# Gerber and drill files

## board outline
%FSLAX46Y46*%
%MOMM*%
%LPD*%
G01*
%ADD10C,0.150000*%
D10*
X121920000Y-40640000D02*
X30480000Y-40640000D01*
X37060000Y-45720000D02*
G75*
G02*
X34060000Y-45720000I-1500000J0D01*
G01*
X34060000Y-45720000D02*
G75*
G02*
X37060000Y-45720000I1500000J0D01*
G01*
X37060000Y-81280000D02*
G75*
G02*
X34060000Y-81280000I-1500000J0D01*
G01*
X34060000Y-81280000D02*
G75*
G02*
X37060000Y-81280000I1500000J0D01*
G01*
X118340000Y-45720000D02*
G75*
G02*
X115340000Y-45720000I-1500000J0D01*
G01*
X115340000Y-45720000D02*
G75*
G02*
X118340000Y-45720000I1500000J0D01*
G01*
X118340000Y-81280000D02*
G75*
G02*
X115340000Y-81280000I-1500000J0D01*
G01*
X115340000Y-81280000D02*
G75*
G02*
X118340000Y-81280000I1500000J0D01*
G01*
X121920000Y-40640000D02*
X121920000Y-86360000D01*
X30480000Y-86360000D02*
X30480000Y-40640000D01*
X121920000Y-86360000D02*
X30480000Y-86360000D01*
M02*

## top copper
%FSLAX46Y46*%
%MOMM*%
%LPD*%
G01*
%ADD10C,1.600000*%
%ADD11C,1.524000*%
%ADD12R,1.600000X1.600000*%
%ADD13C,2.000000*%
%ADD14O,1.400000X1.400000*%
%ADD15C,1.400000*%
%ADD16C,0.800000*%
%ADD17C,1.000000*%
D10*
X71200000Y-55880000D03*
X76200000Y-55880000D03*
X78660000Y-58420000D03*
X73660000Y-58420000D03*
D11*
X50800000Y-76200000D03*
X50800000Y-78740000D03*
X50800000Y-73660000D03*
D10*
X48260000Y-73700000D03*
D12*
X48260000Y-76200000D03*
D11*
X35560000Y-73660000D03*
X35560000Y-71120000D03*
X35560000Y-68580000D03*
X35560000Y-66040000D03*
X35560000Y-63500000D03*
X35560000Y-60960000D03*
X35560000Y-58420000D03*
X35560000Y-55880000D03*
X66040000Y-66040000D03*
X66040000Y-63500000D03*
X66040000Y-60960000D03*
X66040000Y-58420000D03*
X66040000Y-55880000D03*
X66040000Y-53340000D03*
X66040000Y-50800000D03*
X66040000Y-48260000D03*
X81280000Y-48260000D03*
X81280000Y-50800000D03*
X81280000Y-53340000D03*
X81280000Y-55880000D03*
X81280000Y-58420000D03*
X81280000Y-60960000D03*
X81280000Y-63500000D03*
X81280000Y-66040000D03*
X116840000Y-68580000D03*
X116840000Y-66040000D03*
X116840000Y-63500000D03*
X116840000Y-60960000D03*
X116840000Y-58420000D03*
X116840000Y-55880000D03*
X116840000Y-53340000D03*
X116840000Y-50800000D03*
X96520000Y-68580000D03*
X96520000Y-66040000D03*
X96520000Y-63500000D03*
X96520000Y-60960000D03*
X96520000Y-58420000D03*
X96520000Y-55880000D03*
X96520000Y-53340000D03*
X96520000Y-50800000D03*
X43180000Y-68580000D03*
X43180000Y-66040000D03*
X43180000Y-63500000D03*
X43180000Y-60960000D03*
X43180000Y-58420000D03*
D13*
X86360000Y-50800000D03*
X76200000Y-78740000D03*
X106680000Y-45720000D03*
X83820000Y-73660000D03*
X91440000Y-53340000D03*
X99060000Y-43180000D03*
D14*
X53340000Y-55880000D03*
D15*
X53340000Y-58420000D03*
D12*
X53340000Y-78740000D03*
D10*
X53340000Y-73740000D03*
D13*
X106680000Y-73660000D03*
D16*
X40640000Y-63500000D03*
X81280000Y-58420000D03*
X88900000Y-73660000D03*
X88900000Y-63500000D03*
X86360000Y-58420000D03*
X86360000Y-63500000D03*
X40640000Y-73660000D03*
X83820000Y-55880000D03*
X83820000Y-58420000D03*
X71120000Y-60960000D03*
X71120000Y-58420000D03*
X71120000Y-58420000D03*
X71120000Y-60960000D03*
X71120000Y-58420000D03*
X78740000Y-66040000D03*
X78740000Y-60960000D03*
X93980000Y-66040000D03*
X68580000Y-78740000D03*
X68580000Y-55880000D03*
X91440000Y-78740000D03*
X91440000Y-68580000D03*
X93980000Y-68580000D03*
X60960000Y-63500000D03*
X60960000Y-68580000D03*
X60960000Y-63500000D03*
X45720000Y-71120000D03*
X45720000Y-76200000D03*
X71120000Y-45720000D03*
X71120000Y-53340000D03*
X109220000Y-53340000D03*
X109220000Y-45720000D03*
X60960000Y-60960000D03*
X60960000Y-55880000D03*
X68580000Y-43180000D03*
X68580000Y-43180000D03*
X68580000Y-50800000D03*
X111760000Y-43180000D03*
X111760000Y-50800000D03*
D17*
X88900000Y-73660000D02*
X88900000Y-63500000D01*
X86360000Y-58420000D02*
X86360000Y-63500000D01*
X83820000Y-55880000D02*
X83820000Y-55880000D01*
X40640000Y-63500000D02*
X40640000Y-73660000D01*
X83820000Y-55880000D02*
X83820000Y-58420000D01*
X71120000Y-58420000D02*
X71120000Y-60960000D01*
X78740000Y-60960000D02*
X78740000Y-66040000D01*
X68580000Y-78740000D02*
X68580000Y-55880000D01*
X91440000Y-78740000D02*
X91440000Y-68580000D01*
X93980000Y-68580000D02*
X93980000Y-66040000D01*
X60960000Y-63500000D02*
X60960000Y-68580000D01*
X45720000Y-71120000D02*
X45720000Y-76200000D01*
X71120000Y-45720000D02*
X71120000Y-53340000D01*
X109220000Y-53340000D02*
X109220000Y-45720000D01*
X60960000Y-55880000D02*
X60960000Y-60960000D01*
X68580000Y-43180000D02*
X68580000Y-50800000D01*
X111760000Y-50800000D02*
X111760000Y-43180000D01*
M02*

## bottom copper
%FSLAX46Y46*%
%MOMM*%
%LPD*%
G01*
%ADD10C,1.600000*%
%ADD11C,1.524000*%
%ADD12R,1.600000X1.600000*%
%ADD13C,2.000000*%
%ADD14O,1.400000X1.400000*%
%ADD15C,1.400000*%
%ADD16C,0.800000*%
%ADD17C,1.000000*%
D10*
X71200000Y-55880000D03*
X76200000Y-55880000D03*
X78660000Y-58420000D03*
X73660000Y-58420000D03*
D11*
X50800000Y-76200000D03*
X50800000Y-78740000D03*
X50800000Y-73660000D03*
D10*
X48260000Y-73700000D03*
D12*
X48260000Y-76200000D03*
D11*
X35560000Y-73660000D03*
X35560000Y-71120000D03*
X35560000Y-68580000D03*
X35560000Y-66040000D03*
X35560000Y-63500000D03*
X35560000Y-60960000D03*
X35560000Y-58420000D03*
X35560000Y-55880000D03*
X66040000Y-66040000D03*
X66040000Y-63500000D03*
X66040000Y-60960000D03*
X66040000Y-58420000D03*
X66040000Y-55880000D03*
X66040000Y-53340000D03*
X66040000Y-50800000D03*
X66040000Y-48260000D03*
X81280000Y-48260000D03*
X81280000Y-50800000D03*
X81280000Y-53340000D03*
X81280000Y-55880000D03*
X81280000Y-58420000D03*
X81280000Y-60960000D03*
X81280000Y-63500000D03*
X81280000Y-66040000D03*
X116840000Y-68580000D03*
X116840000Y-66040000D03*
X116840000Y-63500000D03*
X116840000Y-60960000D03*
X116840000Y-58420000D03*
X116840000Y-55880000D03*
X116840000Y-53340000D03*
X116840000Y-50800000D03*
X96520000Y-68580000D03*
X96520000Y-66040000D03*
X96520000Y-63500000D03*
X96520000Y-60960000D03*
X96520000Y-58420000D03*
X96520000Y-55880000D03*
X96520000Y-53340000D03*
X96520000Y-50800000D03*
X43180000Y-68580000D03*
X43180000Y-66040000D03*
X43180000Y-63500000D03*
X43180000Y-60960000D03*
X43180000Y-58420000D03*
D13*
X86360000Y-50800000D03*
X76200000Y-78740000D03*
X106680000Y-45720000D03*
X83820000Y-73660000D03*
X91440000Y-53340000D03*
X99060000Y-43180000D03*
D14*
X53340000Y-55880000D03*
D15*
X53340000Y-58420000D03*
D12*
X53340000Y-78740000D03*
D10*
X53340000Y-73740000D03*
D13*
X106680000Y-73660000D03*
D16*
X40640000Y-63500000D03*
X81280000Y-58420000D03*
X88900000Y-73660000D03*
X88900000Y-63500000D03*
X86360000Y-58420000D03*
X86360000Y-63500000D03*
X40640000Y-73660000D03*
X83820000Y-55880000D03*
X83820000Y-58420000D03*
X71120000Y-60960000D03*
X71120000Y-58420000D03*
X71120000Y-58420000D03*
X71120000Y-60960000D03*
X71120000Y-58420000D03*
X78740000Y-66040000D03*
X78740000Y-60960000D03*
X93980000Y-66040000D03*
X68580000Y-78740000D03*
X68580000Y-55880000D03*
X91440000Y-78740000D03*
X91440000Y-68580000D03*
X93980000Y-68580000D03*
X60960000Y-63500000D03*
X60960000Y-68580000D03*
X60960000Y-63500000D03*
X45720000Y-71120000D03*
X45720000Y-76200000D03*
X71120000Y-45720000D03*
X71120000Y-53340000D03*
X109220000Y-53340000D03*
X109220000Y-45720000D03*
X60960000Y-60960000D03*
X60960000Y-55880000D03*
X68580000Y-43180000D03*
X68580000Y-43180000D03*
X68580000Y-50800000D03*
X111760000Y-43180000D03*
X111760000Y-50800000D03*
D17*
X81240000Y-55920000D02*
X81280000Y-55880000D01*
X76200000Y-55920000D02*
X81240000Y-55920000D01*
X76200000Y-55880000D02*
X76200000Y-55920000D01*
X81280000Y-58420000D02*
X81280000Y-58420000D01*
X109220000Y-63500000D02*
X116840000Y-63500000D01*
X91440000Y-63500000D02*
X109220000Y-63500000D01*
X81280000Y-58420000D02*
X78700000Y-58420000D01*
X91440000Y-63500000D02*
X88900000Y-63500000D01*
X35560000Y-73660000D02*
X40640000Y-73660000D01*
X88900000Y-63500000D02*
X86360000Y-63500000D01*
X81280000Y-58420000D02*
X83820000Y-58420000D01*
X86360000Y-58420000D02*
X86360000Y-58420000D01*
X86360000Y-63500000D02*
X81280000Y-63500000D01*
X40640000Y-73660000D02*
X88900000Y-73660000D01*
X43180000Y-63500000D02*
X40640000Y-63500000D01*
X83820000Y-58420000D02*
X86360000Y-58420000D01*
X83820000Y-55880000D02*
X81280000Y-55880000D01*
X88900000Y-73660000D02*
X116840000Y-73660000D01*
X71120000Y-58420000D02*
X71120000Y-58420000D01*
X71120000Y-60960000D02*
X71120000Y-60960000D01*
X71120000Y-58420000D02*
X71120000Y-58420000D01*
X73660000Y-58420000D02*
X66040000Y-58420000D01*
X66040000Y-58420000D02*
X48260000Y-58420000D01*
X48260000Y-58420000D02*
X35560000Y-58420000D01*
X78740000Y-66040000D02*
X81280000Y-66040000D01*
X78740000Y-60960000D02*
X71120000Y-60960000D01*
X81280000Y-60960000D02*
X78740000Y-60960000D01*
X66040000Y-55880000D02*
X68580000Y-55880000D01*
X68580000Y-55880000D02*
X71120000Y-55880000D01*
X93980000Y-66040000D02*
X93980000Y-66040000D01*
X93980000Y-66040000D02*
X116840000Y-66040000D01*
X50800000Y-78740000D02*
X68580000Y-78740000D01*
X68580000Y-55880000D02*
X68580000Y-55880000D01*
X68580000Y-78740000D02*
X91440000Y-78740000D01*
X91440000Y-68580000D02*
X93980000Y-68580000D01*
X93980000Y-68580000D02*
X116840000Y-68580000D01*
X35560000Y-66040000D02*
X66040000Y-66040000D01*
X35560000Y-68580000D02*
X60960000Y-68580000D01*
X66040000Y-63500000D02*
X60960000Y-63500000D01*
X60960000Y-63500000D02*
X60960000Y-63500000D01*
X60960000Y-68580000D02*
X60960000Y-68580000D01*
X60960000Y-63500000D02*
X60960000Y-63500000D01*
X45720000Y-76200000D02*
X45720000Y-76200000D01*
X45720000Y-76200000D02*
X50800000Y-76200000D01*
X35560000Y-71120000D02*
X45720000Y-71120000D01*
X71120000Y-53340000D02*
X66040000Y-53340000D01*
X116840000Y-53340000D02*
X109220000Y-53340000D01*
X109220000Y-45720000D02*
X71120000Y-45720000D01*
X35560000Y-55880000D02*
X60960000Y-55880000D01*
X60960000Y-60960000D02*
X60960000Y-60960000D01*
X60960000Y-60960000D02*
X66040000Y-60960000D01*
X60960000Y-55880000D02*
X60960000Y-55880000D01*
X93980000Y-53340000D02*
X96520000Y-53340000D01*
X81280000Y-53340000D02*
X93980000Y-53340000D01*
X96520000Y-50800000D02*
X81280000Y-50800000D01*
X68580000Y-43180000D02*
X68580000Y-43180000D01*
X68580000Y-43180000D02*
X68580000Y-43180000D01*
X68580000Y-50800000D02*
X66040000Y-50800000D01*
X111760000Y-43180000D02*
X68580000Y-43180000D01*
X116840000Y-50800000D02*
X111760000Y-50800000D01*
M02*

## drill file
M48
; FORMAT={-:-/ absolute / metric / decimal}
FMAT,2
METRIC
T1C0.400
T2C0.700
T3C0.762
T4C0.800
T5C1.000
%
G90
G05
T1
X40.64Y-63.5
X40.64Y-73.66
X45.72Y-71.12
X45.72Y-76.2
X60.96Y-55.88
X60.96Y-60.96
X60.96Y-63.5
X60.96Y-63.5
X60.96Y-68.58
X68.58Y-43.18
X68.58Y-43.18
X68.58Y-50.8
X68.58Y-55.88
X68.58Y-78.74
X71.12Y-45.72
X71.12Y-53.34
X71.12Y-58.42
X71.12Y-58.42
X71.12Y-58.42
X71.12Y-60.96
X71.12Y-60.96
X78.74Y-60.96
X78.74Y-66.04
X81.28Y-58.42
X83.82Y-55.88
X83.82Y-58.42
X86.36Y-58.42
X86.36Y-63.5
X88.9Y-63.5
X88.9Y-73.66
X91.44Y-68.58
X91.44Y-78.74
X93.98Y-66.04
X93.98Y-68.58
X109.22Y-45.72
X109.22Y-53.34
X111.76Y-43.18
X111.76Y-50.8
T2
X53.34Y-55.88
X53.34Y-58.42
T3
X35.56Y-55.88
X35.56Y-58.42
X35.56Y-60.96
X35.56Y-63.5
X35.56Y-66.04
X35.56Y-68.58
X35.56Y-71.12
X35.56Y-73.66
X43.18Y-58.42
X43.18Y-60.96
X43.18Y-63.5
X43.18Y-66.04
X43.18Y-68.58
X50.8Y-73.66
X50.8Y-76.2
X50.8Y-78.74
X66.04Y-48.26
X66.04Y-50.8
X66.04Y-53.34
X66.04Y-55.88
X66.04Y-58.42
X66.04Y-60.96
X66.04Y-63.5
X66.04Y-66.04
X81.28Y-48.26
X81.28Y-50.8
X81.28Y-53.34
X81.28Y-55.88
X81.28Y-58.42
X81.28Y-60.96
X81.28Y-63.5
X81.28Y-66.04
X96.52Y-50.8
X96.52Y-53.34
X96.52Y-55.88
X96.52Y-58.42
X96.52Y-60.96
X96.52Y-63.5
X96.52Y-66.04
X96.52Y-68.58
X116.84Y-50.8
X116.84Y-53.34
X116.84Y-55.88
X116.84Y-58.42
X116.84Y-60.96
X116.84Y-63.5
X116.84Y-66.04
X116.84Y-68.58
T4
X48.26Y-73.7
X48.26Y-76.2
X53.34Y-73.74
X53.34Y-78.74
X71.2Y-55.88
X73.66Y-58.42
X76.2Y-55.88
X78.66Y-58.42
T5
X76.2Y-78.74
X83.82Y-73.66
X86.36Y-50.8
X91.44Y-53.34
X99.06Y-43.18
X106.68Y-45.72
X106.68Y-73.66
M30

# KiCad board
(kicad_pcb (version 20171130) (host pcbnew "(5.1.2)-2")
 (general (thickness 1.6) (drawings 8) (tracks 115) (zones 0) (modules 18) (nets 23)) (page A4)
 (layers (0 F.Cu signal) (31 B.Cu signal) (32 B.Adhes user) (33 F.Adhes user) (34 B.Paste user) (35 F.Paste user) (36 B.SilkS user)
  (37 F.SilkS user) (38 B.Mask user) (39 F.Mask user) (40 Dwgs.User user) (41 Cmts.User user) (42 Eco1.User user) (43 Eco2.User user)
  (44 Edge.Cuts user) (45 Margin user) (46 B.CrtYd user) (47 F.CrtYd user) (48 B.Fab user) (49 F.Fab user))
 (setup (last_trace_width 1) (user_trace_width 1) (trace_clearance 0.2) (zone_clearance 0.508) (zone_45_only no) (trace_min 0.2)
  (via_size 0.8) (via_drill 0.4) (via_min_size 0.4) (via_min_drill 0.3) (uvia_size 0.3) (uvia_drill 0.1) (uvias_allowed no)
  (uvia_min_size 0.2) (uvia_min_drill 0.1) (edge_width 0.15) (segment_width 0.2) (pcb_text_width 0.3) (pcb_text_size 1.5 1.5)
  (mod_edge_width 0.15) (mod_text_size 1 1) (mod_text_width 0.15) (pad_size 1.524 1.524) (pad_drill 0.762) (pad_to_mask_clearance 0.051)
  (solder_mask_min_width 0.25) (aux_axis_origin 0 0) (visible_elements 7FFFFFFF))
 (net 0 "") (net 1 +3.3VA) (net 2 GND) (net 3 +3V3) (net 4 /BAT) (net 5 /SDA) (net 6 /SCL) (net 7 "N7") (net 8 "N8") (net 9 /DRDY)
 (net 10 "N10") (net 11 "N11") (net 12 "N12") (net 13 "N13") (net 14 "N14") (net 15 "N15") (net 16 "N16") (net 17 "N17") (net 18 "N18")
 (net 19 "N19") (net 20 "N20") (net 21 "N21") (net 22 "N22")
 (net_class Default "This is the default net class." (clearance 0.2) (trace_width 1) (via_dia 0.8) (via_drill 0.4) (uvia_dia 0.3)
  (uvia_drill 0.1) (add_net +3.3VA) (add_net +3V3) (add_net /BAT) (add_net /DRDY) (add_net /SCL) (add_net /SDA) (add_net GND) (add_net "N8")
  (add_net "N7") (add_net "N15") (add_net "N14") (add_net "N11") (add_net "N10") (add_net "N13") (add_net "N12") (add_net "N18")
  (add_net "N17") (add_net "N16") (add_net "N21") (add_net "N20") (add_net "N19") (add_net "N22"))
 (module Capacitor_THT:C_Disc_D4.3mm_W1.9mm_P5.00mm (layer F.Cu) (at 76.2 55.88 180)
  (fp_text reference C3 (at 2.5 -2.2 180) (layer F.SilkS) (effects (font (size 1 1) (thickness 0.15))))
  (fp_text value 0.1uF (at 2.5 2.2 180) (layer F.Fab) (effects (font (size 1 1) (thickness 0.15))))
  (pad 2 thru_hole circle (at 5 0 180) (size 1.6 1.6) (drill 0.8) (layers *.Cu *.Mask) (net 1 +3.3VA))
  (pad 1 thru_hole circle (at 0 0 180) (size 1.6 1.6) (drill 0.8) (layers *.Cu *.Mask) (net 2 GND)))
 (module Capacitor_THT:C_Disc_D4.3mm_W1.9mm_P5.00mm (layer F.Cu) (at 73.66 58.42)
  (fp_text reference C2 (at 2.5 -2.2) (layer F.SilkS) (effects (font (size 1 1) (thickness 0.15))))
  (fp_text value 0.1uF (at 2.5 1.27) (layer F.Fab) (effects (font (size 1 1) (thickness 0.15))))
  (pad 2 thru_hole circle (at 5 0) (size 1.6 1.6) (drill 0.8) (layers *.Cu *.Mask) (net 2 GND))
  (pad 1 thru_hole circle (at 0 0) (size 1.6 1.6) (drill 0.8) (layers *.Cu *.Mask) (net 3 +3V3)))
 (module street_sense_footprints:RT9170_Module (layer F.Cu) (at 53.34 76.2 270)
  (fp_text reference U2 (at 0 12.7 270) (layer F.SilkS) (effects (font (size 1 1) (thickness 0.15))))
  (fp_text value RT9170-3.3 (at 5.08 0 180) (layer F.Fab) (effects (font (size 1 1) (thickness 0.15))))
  (pad 3 thru_hole circle (at 0 2.54 270) (size 1.524 1.524) (drill 0.762) (layers *.Cu *.Mask) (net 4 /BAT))
  (pad 2 thru_hole circle (at 2.54 2.54 270) (size 1.524 1.524) (drill 0.762) (layers *.Cu *.Mask) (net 1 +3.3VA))
  (pad 1 thru_hole circle (at -2.54 2.54 270) (size 1.524 1.524) (drill 0.762) (layers *.Cu *.Mask) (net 2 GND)))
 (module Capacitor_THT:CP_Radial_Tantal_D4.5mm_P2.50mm (layer F.Cu) (at 48.26 76.2 90)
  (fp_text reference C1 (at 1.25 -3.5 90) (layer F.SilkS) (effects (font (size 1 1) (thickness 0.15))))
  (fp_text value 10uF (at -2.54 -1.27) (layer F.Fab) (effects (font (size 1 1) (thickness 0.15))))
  (pad 2 thru_hole circle (at 2.5 0 90) (size 1.6 1.6) (drill 0.8) (layers *.Cu *.Mask) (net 2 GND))
  (pad 1 thru_hole rect (at 0 0 90) (size 1.6 1.6) (drill 0.8) (layers *.Cu *.Mask) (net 4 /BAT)))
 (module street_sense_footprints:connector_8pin (layer F.Cu) (at 35.56 53.34)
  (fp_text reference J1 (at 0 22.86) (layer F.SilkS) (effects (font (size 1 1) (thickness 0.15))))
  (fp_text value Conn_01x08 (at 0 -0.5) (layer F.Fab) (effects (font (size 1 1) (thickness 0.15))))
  (pad 8 thru_hole circle (at 0 20.32) (size 1.524 1.524) (drill 0.762) (layers *.Cu *.Mask) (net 2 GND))
  (pad 7 thru_hole circle (at 0 17.78) (size 1.524 1.524) (drill 0.762) (layers *.Cu *.Mask) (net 4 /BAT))
  (pad 6 thru_hole circle (at 0 15.24) (size 1.524 1.524) (drill 0.762) (layers *.Cu *.Mask) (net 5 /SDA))
  (pad 5 thru_hole circle (at 0 12.7) (size 1.524 1.524) (drill 0.762) (layers *.Cu *.Mask) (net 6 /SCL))
  (pad 4 thru_hole circle (at 0 10.16) (size 1.524 1.524) (drill 0.762) (layers *.Cu *.Mask) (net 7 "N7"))
  (pad 3 thru_hole circle (at 0 7.62) (size 1.524 1.524) (drill 0.762) (layers *.Cu *.Mask) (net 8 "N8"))
  (pad 2 thru_hole circle (at 0 5.08) (size 1.524 1.524) (drill 0.762) (layers *.Cu *.Mask) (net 3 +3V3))
  (pad 1 thru_hole circle (at 0 2.54) (size 1.524 1.524) (drill 0.762) (layers *.Cu *.Mask) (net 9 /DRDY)))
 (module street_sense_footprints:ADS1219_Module (layer F.Cu) (at 76.2 68.58 180)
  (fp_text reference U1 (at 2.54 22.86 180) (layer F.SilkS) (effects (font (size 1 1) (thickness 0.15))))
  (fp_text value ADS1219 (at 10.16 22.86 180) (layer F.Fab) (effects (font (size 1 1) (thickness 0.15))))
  (pad 16 thru_hole circle (at 10.16 2.54 180) (size 1.524 1.524) (drill 0.762) (layers *.Cu *.Mask) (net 6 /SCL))
  (pad 15 thru_hole circle (at 10.16 5.08 180) (size 1.524 1.524) (drill 0.762) (layers *.Cu *.Mask) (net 5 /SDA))
  (pad 14 thru_hole circle (at 10.16 7.62 180) (size 1.524 1.524) (drill 0.762) (layers *.Cu *.Mask) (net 9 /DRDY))
  (pad 13 thru_hole circle (at 10.16 10.16 180) (size 1.524 1.524) (drill 0.762) (layers *.Cu *.Mask) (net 3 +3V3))
  (pad 12 thru_hole circle (at 10.16 12.7 180) (size 1.524 1.524) (drill 0.762) (layers *.Cu *.Mask) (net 1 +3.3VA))
  (pad 11 thru_hole circle (at 10.16 15.24 180) (size 1.524 1.524) (drill 0.762) (layers *.Cu *.Mask) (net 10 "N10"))
  (pad 10 thru_hole circle (at 10.16 17.78 180) (size 1.524 1.524) (drill 0.762) (layers *.Cu *.Mask) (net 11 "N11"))
  (pad 9 thru_hole circle (at 10.16 20.32 180) (size 1.524 1.524) (drill 0.762) (layers *.Cu *.Mask) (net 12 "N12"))
  (pad 8 thru_hole circle (at -5.08 20.32 180) (size 1.524 1.524) (drill 0.762) (layers *.Cu *.Mask) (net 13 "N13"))
  (pad 7 thru_hole circle (at -5.08 17.78 180) (size 1.524 1.524) (drill 0.762) (layers *.Cu *.Mask) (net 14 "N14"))
  (pad 6 thru_hole circle (at -5.08 15.24 180) (size 1.524 1.524) (drill 0.762) (layers *.Cu *.Mask) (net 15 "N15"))
  (pad 5 thru_hole circle (at -5.08 12.7 180) (size 1.524 1.524) (drill 0.762) (layers *.Cu *.Mask) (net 2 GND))
  (pad 4 thru_hole circle (at -5.08 10.16 180) (size 1.524 1.524) (drill 0.762) (layers *.Cu *.Mask) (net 2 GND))
  (pad 3 thru_hole circle (at -5.08 7.62 180) (size 1.524 1.524) (drill 0.762) (layers *.Cu *.Mask) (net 3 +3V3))
  (pad 2 thru_hole circle (at -5.08 5.08 180) (size 1.524 1.524) (drill 0.762) (layers *.Cu *.Mask) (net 2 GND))
  (pad 1 thru_hole circle (at -5.08 2.54 180) (size 1.524 1.524) (drill 0.762) (layers *.Cu *.Mask) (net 3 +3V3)))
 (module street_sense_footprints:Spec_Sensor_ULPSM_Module (layer F.Cu) (at 119.38 60.96 270)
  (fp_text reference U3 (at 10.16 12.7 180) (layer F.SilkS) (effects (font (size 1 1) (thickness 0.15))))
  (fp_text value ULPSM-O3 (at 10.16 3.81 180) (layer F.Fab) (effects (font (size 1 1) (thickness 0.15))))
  (pad 8 thru_hole circle (at 7.62 2.54 270) (size 1.524 1.524) (drill 0.762) (layers *.Cu *.Mask) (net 1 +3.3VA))
  (pad 7 thru_hole circle (at 5.08 2.54 270) (size 1.524 1.524) (drill 0.762) (layers *.Cu *.Mask) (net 1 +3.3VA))
  (pad 6 thru_hole circle (at 2.54 2.54 270) (size 1.524 1.524) (drill 0.762) (layers *.Cu *.Mask) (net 2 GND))
  (pad 5 thru_hole circle (at 0 2.54 270) (size 1.524 1.524) (drill 0.762) (layers *.Cu *.Mask) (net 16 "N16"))
  (pad 4 thru_hole circle (at -2.54 2.54 270) (size 1.524 1.524) (drill 0.762) (layers *.Cu *.Mask) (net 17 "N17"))
  (pad 3 thru_hole circle (at -5.08 2.54 270) (size 1.524 1.524) (drill 0.762) (layers *.Cu *.Mask) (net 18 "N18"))
  (pad 2 thru_hole circle (at -7.62 2.54 270) (size 1.524 1.524) (drill 0.762) (layers *.Cu *.Mask) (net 10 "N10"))
  (pad 1 thru_hole circle (at -10.16 2.54 270) (size 1.524 1.524) (drill 0.762) (layers *.Cu *.Mask) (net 11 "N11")))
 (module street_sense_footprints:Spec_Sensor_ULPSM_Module (layer F.Cu) (at 99.06 60.96 270)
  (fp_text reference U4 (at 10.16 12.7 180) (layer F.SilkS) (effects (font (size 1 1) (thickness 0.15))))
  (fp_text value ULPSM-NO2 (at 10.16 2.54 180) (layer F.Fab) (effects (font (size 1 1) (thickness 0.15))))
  (pad 8 thru_hole circle (at 7.62 2.54 270) (size 1.524 1.524) (drill 0.762) (layers *.Cu *.Mask) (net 1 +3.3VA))
  (pad 7 thru_hole circle (at 5.08 2.54 270) (size 1.524 1.524) (drill 0.762) (layers *.Cu *.Mask) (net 1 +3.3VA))
  (pad 6 thru_hole circle (at 2.54 2.54 270) (size 1.524 1.524) (drill 0.762) (layers *.Cu *.Mask) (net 2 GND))
  (pad 5 thru_hole circle (at 0 2.54 270) (size 1.524 1.524) (drill 0.762) (layers *.Cu *.Mask) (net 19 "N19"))
  (pad 4 thru_hole circle (at -2.54 2.54 270) (size 1.524 1.524) (drill 0.762) (layers *.Cu *.Mask) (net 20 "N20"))
  (pad 3 thru_hole circle (at -5.08 2.54 270) (size 1.524 1.524) (drill 0.762) (layers *.Cu *.Mask) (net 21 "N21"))
  (pad 2 thru_hole circle (at -7.62 2.54 270) (size 1.524 1.524) (drill 0.762) (layers *.Cu *.Mask) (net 15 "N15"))
  (pad 1 thru_hole circle (at -10.16 2.54 270) (size 1.524 1.524) (drill 0.762) (layers *.Cu *.Mask) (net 14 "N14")))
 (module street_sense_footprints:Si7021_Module (layer F.Cu) (at 53.34 63.5 270)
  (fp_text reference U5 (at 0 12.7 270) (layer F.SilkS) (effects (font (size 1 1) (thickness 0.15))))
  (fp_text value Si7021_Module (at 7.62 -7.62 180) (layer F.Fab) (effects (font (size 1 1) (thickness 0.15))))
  (pad 5 thru_hole circle (at 5.08 10.16 270) (size 1.524 1.524) (drill 0.762) (layers *.Cu *.Mask) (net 5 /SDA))
  (pad 4 thru_hole circle (at 2.54 10.16 270) (size 1.524 1.524) (drill 0.762) (layers *.Cu *.Mask) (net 6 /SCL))
  (pad 3 thru_hole circle (at 0 10.16 270) (size 1.524 1.524) (drill 0.762) (layers *.Cu *.Mask) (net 2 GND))
  (pad 2 thru_hole circle (at -2.54 10.16 270) (size 1.524 1.524) (drill 0.762) (layers *.Cu *.Mask) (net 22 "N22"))
  (pad 1 thru_hole circle (at -5.08 10.16 270) (size 1.524 1.524) (drill 0.762) (layers *.Cu *.Mask) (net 3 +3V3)))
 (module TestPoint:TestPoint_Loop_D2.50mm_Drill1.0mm (layer F.Cu) (at 86.36 50.8)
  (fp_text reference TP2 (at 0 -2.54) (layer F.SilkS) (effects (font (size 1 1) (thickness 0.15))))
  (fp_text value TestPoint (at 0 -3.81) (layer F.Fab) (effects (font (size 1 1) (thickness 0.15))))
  (pad 1 thru_hole circle (at 0 0) (size 2 2) (drill 1) (layers *.Cu *.Mask) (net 14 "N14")))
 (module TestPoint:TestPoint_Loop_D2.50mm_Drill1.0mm (layer F.Cu) (at 76.2 78.74)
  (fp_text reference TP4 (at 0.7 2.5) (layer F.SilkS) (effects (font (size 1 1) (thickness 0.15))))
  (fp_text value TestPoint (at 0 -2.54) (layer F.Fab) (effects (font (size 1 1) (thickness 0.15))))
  (pad 1 thru_hole circle (at 0 0) (size 2 2) (drill 1) (layers *.Cu *.Mask) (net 1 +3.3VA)))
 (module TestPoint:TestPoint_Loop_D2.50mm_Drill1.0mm (layer F.Cu) (at 106.68 45.72)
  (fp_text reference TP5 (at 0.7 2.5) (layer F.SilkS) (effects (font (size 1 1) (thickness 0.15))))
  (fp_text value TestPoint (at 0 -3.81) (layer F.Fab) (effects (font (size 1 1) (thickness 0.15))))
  (pad 1 thru_hole circle (at 0 0) (size 2 2) (drill 1) (layers *.Cu *.Mask) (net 10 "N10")))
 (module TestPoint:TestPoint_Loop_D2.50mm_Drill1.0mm (layer F.Cu) (at 83.82 73.66)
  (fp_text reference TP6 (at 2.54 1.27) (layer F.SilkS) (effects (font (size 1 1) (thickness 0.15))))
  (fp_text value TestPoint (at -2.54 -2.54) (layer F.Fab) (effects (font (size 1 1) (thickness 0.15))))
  (pad 1 thru_hole circle (at 0 0) (size 2 2) (drill 1) (layers *.Cu *.Mask) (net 2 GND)))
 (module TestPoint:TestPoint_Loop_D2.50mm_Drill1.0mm (layer F.Cu) (at 91.44 53.34)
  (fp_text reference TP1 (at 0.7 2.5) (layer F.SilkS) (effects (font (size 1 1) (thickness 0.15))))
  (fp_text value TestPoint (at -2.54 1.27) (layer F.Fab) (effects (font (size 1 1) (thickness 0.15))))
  (pad 1 thru_hole circle (at 0 0) (size 2 2) (drill 1) (layers *.Cu *.Mask) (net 15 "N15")))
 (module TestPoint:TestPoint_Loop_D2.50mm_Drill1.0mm (layer F.Cu) (at 99.06 43.18)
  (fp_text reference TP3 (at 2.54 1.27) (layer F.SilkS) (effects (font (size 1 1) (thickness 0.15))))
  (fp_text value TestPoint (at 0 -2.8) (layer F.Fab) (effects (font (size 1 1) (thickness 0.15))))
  (pad 1 thru_hole circle (at 0 0) (size 2 2) (drill 1) (layers *.Cu *.Mask) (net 11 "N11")))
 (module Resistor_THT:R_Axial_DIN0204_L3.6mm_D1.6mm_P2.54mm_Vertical (layer F.Cu) (at 53.34 58.42 90)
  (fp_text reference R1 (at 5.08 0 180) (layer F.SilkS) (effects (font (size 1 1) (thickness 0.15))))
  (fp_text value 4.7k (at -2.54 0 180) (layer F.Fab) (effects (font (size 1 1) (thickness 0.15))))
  (pad 2 thru_hole oval (at 2.54 0 90) (size 1.4 1.4) (drill 0.7) (layers *.Cu *.Mask) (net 9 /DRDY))
  (pad 1 thru_hole circle (at 0 0 90) (size 1.4 1.4) (drill 0.7) (layers *.Cu *.Mask) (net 3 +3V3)))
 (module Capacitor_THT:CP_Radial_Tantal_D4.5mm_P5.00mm (layer F.Cu) (at 53.34 78.74 90)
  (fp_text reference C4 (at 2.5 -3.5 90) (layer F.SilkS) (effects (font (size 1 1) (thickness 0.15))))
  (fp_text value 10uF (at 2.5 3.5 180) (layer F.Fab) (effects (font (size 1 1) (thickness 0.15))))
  (pad 1 thru_hole rect (at 0 0 90) (size 1.6 1.6) (drill 0.8) (layers *.Cu *.Mask) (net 1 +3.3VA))
  (pad 2 thru_hole circle (at 5 0 90) (size 1.6 1.6) (drill 0.8) (layers *.Cu *.Mask) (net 2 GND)))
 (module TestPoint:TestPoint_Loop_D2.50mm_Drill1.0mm (layer F.Cu) (at 106.68 73.66)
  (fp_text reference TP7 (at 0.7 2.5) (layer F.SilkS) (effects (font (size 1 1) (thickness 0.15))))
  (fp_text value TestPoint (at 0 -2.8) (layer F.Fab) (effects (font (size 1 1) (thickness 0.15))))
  (pad 1 thru_hole circle (at 0 0) (size 2 2) (drill 1) (layers *.Cu *.Mask) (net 2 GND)))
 (gr_line (start 121.92 40.64) (end 30.48 40.64) (layer Edge.Cuts) (width 0.15))
 (gr_circle (center 35.56 45.72) (end 37.06 45.72) (layer Edge.Cuts) (width 0.15))
 (gr_circle (center 35.56 81.28) (end 37.06 81.28) (layer Edge.Cuts) (width 0.15))
 (gr_circle (center 116.84 45.72) (end 118.34 45.72) (layer Edge.Cuts) (width 0.15))
 (gr_circle (center 116.84 81.28) (end 118.34 81.28) (layer Edge.Cuts) (width 0.15))
 (gr_line (start 121.92 40.64) (end 121.92 86.36) (layer Edge.Cuts) (width 0.15))
 (gr_line (start 30.48 86.36) (end 30.48 40.64) (layer Edge.Cuts) (width 0.15))
 (gr_line (start 121.92 86.36) (end 30.48 86.36) (layer Edge.Cuts) (width 0.15))
 (via (at 40.64 63.5) (size 0.8) (drill 0.4) (layers F.Cu B.Cu) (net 2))
 (segment (start 81.24 55.92) (end 81.28 55.88) (width 1) (layer B.Cu) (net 2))
 (segment (start 76.2 55.92) (end 81.24 55.92) (width 1) (layer B.Cu) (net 2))
 (segment (start 76.2 55.88) (end 76.2 55.92) (width 1) (layer B.Cu) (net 2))
 (segment (start 81.28 58.42) (end 81.28 58.42) (width 1) (layer B.Cu) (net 2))
 (segment (start 109.22 63.5) (end 116.84 63.5) (width 1) (layer B.Cu) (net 2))
 (segment (start 91.44 63.5) (end 109.22 63.5) (width 1) (layer B.Cu) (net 2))
 (segment (start 81.28 58.42) (end 78.7 58.42) (width 1) (layer B.Cu) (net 2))
 (via (at 81.28 58.42) (size 0.8) (drill 0.4) (layers F.Cu B.Cu) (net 2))
 (segment (start 91.44 63.5) (end 88.9 63.5) (width 1) (layer B.Cu) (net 2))
 (via (at 88.9 73.66) (size 0.8) (drill 0.4) (layers F.Cu B.Cu) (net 2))
 (segment (start 35.56 73.66) (end 40.64 73.66) (width 1) (layer B.Cu) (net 2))
 (segment (start 88.9 73.66) (end 88.9 63.5) (width 1) (layer F.Cu) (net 2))
 (segment (start 88.9 63.5) (end 86.36 63.5) (width 1) (layer B.Cu) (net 2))
 (via (at 88.9 63.5) (size 0.8) (drill 0.4) (layers F.Cu B.Cu) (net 2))
 (segment (start 81.28 58.42) (end 83.82 58.42) (width 1) (layer B.Cu) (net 2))
 (segment (start 86.36 58.42) (end 86.36 58.42) (width 1) (layer B.Cu) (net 2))
 (via (at 86.36 58.42) (size 0.8) (drill 0.4) (layers F.Cu B.Cu) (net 2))
 (segment (start 86.36 63.5) (end 81.28 63.5) (width 1) (layer B.Cu) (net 2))
 (via (at 86.36 63.5) (size 0.8) (drill 0.4) (layers F.Cu B.Cu) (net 2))
 (segment (start 86.36 58.42) (end 86.36 63.5) (width 1) (layer F.Cu) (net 2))
 (segment (start 83.82 55.88) (end 83.82 55.88) (width 1) (layer F.Cu) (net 2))
 (segment (start 40.64 73.66) (end 88.9 73.66) (width 1) (layer B.Cu) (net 2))
 (via (at 40.64 73.66) (size 0.8) (drill 0.4) (layers F.Cu B.Cu) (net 2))
 (segment (start 43.18 63.5) (end 40.64 63.5) (width 1) (layer B.Cu) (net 2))
 (segment (start 40.64 63.5) (end 40.64 73.66) (width 1) (layer F.Cu) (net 2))
 (segment (start 83.82 55.88) (end 83.82 58.42) (width 1) (layer F.Cu) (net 2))
 (via (at 83.82 55.88) (size 0.8) (drill 0.4) (layers F.Cu B.Cu) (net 2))
 (segment (start 83.82 58.42) (end 86.36 58.42) (width 1) (layer B.Cu) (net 2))
 (via (at 83.82 58.42) (size 0.8) (drill 0.4) (layers F.Cu B.Cu) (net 2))
 (segment (start 83.82 55.88) (end 81.28 55.88) (width 1) (layer B.Cu) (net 2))
 (segment (start 88.9 73.66) (end 116.84 73.66) (width 1) (layer B.Cu) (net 2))
 (via (at 71.12 60.96) (size 0.8) (drill 0.4) (layers F.Cu B.Cu) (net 3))
 (via (at 71.12 58.42) (size 0.8) (drill 0.4) (layers F.Cu B.Cu) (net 3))
 (segment (start 71.12 58.42) (end 71.12 58.42) (width 1) (layer B.Cu) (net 3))
 (via (at 71.12 58.42) (size 0.8) (drill 0.4) (layers F.Cu B.Cu) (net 3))
 (segment (start 71.12 60.96) (end 71.12 60.96) (width 1) (layer B.Cu) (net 3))
 (via (at 71.12 60.96) (size 0.8) (drill 0.4) (layers F.Cu B.Cu) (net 3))
 (segment (start 71.12 58.42) (end 71.12 58.42) (width 1) (layer B.Cu) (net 3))
 (via (at 71.12 58.42) (size 0.8) (drill 0.4) (layers F.Cu B.Cu) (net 3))
 (segment (start 71.12 58.42) (end 71.12 60.96) (width 1) (layer F.Cu) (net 3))
 (segment (start 73.66 58.42) (end 66.04 58.42) (width 1) (layer B.Cu) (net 3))
 (segment (start 66.04 58.42) (end 48.26 58.42) (width 1) (layer B.Cu) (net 3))
 (segment (start 48.26 58.42) (end 35.56 58.42) (width 1) (layer B.Cu) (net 3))
 (via (at 78.74 66.04) (size 0.8) (drill 0.4) (layers F.Cu B.Cu) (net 3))
 (segment (start 78.74 60.96) (end 78.74 66.04) (width 1) (layer F.Cu) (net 3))
 (segment (start 78.74 66.04) (end 81.28 66.04) (width 1) (layer B.Cu) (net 3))
 (via (at 78.74 60.96) (size 0.8) (drill 0.4) (layers F.Cu B.Cu) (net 3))
 (segment (start 78.74 60.96) (end 71.12 60.96) (width 1) (layer B.Cu) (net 3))
 (segment (start 81.28 60.96) (end 78.74 60.96) (width 1) (layer B.Cu) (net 3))
 (segment (start 66.04 55.88) (end 68.58 55.88) (width 1) (layer B.Cu) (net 1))
 (segment (start 68.58 55.88) (end 71.12 55.88) (width 1) (layer B.Cu) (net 1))
 (segment (start 93.98 66.04) (end 93.98 66.04) (width 1) (layer B.Cu) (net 1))
 (segment (start 93.98 66.04) (end 116.84 66.04) (width 1) (layer B.Cu) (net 1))
 (via (at 93.98 66.04) (size 0.8) (drill 0.4) (layers F.Cu B.Cu) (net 1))
 (segment (start 50.8 78.74) (end 68.58 78.74) (width 1) (layer B.Cu) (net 1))
 (via (at 68.58 78.74) (size 0.8) (drill 0.4) (layers F.Cu B.Cu) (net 1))
 (segment (start 68.58 55.88) (end 68.58 55.88) (width 1) (layer B.Cu) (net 1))
 (via (at 68.58 55.88) (size 0.8) (drill 0.4) (layers F.Cu B.Cu) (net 1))
 (segment (start 68.58 78.74) (end 68.58 55.88) (width 1) (layer F.Cu) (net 1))
 (via (at 91.44 78.74) (size 0.8) (drill 0.4) (layers F.Cu B.Cu) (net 1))
 (segment (start 68.58 78.74) (end 91.44 78.74) (width 1) (layer B.Cu) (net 1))
 (via (at 91.44 68.58) (size 0.8) (drill 0.4) (layers F.Cu B.Cu) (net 1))
 (segment (start 91.44 68.58) (end 93.98 68.58) (width 1) (layer B.Cu) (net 1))
 (segment (start 91.44 78.74) (end 91.44 68.58) (width 1) (layer F.Cu) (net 1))
 (segment (start 93.98 68.58) (end 93.98 66.04) (width 1) (layer F.Cu) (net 1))
 (segment (start 93.98 68.58) (end 116.84 68.58) (width 1) (layer B.Cu) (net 1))
 (via (at 93.98 68.58) (size 0.8) (drill 0.4) (layers F.Cu B.Cu) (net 1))
 (segment (start 35.56 66.04) (end 66.04 66.04) (width 1) (layer B.Cu) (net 6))
 (segment (start 35.56 68.58) (end 60.96 68.58) (width 1) (layer B.Cu) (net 5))
 (segment (start 66.04 63.5) (end 60.96 63.5) (width 1) (layer B.Cu) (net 5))
 (segment (start 60.96 63.5) (end 60.96 63.5) (width 1) (layer B.Cu) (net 5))
 (via (at 60.96 63.5) (size 0.8) (drill 0.4) (layers F.Cu B.Cu) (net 5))
 (segment (start 60.96 68.58) (end 60.96 68.58) (width 1) (layer B.Cu) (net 5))
 (via (at 60.96 68.58) (size 0.8) (drill 0.4) (layers F.Cu B.Cu) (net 5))
 (segment (start 60.96 63.5) (end 60.96 63.5) (width 1) (layer B.Cu) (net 5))
 (via (at 60.96 63.5) (size 0.8) (drill 0.4) (layers F.Cu B.Cu) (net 5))
 (segment (start 60.96 63.5) (end 60.96 68.58) (width 1) (layer F.Cu) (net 5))
 (via (at 45.72 71.12) (size 0.8) (drill 0.4) (layers F.Cu B.Cu) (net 4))
 (segment (start 45.72 76.2) (end 45.72 76.2) (width 1) (layer B.Cu) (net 4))
 (segment (start 45.72 76.2) (end 50.8 76.2) (width 1) (layer B.Cu) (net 4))
 (via (at 45.72 76.2) (size 0.8) (drill 0.4) (layers F.Cu B.Cu) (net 4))
 (segment (start 35.56 71.12) (end 45.72 71.12) (width 1) (layer B.Cu) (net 4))
 (segment (start 45.72 71.12) (end 45.72 76.2) (width 1) (layer F.Cu) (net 4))
 (via (at 71.12 45.72) (size 0.8) (drill 0.4) (layers F.Cu B.Cu) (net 10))
 (via (at 71.12 53.34) (size 0.8) (drill 0.4) (layers F.Cu B.Cu) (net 10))
 (segment (start 71.12 45.72) (end 71.12 53.34) (width 1) (layer F.Cu) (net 10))
 (segment (start 71.12 53.34) (end 66.04 53.34) (width 1) (layer B.Cu) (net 10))
 (segment (start 116.84 53.34) (end 109.22 53.34) (width 1) (layer B.Cu) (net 10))
 (via (at 109.22 53.34) (size 0.8) (drill 0.4) (layers F.Cu B.Cu) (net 10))
 (via (at 109.22 45.72) (size 0.8) (drill 0.4) (layers F.Cu B.Cu) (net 10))
 (segment (start 109.22 53.34) (end 109.22 45.72) (width 1) (layer F.Cu) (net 10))
 (segment (start 109.22 45.72) (end 71.12 45.72) (width 1) (layer B.Cu) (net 10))
 (segment (start 35.56 55.88) (end 60.96 55.88) (width 1) (layer B.Cu) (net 9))
 (segment (start 60.96 60.96) (end 60.96 60.96) (width 1) (layer B.Cu) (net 9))
 (segment (start 60.96 60.96) (end 66.04 60.96) (width 1) (layer B.Cu) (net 9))
 (via (at 60.96 60.96) (size 0.8) (drill 0.4) (layers F.Cu B.Cu) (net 9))
 (segment (start 60.96 55.88) (end 60.96 55.88) (width 1) (layer B.Cu) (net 9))
 (via (at 60.96 55.88) (size 0.8) (drill 0.4) (layers F.Cu B.Cu) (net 9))
 (segment (start 60.96 55.88) (end 60.96 60.96) (width 1) (layer F.Cu) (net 9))
 (segment (start 93.98 53.34) (end 96.52 53.34) (width 1) (layer B.Cu) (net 15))
 (segment (start 81.28 53.34) (end 93.98 53.34) (width 1) (layer B.Cu) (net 15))
 (segment (start 96.52 50.8) (end 81.28 50.8) (width 1) (layer B.Cu) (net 14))
 (segment (start 68.58 43.18) (end 68.58 43.18) (width 1) (layer B.Cu) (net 11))
 (via (at 68.58 43.18) (size 0.8) (drill 0.4) (layers F.Cu B.Cu) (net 11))
 (segment (start 68.58 43.18) (end 68.58 43.18) (width 1) (layer B.Cu) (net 11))
 (via (at 68.58 43.18) (size 0.8) (drill 0.4) (layers F.Cu B.Cu) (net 11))
 (via (at 68.58 50.8) (size 0.8) (drill 0.4) (layers F.Cu B.Cu) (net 11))
 (segment (start 68.58 43.18) (end 68.58 50.8) (width 1) (layer F.Cu) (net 11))
 (segment (start 68.58 50.8) (end 66.04 50.8) (width 1) (layer B.Cu) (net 11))
 (via (at 111.76 43.18) (size 0.8) (drill 0.4) (layers F.Cu B.Cu) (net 11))
 (segment (start 111.76 43.18) (end 68.58 43.18) (width 1) (layer B.Cu) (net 11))
 (via (at 111.76 50.8) (size 0.8) (drill 0.4) (layers F.Cu B.Cu) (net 11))
 (segment (start 111.76 50.8) (end 111.76 43.18) (width 1) (layer F.Cu) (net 11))
 (segment (start 116.84 50.8) (end 111.76 50.8) (width 1) (layer B.Cu) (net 11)))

